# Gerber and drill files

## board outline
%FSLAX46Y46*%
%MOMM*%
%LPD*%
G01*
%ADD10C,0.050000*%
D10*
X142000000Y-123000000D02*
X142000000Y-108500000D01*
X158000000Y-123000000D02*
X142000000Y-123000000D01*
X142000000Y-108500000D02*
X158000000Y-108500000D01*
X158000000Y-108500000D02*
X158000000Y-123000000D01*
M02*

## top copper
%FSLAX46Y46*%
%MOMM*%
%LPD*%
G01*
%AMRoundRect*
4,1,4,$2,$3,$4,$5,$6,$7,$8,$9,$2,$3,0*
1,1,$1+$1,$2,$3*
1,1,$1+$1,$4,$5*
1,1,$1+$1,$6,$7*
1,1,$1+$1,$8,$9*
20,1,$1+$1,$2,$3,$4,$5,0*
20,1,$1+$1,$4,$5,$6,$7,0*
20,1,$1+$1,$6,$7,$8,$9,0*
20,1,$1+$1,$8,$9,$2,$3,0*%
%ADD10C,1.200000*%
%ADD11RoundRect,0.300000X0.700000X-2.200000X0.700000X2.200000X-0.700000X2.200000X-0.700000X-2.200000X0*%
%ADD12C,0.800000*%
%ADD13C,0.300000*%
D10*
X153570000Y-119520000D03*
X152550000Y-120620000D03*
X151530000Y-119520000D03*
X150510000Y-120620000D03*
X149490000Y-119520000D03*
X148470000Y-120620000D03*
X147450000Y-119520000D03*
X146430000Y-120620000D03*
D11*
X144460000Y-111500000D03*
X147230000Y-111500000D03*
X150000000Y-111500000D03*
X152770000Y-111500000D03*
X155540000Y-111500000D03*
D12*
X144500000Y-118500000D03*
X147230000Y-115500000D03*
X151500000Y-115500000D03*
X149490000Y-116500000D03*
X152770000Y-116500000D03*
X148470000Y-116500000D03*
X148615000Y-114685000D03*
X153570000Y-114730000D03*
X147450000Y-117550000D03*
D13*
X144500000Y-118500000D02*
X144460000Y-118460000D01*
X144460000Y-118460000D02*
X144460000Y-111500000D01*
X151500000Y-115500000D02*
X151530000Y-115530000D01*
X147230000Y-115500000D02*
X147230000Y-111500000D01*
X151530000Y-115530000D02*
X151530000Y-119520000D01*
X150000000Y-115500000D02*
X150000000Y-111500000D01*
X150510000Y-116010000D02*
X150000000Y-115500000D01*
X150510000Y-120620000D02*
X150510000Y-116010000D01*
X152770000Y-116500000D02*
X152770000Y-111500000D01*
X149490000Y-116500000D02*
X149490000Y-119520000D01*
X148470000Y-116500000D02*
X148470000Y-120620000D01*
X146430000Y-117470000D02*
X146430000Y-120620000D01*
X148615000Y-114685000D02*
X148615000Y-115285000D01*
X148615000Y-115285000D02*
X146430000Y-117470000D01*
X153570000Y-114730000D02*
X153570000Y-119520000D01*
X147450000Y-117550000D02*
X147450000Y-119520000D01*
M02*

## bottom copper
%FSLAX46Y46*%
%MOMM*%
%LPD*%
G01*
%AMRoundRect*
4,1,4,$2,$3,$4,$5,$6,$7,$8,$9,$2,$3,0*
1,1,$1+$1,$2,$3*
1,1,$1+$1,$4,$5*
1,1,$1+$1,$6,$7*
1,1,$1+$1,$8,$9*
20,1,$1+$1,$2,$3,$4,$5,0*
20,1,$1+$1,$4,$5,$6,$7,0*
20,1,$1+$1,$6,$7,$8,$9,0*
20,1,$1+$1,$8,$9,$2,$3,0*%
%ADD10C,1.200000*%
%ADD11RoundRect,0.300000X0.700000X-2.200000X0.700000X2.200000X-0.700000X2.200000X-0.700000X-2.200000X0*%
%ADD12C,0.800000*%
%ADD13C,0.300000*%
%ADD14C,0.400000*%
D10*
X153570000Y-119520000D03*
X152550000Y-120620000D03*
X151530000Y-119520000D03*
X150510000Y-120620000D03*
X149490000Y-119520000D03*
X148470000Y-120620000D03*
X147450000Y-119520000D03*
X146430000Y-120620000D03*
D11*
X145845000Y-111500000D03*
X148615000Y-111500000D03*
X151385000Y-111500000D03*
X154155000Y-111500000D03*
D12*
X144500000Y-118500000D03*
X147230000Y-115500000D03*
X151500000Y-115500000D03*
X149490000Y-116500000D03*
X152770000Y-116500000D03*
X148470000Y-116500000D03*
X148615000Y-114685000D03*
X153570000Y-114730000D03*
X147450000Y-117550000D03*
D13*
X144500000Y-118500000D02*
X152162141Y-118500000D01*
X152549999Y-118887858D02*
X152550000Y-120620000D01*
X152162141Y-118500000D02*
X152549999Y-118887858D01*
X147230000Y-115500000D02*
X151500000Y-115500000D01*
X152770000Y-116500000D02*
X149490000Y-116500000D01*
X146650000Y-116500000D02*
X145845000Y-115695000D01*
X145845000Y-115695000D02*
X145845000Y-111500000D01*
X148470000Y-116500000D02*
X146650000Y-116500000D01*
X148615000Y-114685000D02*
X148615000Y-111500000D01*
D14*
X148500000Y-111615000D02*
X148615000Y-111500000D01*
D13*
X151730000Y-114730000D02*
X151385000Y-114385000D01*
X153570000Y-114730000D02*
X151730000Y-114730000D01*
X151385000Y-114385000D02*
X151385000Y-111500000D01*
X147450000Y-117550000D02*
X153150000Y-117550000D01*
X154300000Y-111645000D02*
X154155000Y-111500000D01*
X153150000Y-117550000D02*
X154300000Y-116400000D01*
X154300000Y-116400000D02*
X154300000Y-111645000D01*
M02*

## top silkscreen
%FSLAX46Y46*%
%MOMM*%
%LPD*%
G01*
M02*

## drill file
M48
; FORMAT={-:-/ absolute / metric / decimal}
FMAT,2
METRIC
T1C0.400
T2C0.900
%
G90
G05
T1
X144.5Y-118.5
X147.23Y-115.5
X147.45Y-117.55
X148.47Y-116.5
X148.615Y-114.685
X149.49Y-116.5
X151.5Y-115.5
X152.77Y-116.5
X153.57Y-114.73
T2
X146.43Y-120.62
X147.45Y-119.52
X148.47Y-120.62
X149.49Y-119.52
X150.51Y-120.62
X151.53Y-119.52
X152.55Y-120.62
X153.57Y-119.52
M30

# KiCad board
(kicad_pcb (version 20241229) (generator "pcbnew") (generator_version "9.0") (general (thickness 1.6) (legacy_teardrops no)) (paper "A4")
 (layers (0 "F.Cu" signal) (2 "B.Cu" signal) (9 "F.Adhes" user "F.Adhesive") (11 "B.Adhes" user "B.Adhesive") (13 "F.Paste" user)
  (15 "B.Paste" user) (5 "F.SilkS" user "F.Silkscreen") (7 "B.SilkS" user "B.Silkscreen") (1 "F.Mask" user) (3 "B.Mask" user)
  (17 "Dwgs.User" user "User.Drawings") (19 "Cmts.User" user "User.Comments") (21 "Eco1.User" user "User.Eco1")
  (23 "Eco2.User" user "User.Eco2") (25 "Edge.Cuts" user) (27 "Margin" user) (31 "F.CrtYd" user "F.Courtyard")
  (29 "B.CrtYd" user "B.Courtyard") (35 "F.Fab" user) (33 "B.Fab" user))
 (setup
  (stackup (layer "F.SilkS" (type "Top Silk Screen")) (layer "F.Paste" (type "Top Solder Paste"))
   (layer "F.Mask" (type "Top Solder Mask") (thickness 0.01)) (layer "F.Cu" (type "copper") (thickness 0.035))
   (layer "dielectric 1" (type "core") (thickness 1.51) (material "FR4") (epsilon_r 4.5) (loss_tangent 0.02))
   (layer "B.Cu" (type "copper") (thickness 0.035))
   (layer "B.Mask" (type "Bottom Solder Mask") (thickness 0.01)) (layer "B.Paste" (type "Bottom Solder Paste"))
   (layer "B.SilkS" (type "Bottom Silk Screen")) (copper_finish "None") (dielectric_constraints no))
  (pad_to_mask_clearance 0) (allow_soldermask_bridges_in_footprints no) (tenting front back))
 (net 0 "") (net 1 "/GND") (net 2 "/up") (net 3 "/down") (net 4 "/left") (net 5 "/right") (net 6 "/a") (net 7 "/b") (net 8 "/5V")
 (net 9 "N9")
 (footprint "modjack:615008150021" (layer "F.Cu") (at 150 122.5)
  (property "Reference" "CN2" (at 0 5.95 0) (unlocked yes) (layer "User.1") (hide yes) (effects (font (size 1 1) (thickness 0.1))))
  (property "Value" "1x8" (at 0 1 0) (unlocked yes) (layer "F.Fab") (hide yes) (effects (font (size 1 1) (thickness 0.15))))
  (pad "1" thru_hole circle (at 3.57 -2.98) (size 1.2 1.2) (drill 0.9) (layers "*.Cu" "*.Mask") (remove_unused_layers no) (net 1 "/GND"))
  (pad "2" thru_hole circle (at 2.55 -1.88) (size 1.2 1.2) (drill 0.9) (layers "*.Cu" "*.Mask") (remove_unused_layers no) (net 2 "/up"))
  (pad "3" thru_hole circle (at 1.53 -2.98) (size 1.2 1.2) (drill 0.9) (layers "*.Cu" "*.Mask") (remove_unused_layers no) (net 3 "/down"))
  (pad "4" thru_hole circle (at 0.51 -1.88) (size 1.2 1.2) (drill 0.9) (layers "*.Cu" "*.Mask") (remove_unused_layers no) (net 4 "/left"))
  (pad "5" thru_hole circle (at -0.51 -2.98) (size 1.2 1.2) (drill 0.9) (layers "*.Cu" "*.Mask") (remove_unused_layers no) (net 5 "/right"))
  (pad "6" thru_hole circle (at -1.53 -1.88) (size 1.2 1.2) (drill 0.9) (layers "*.Cu" "*.Mask") (remove_unused_layers no) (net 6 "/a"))
  (pad "7" thru_hole circle (at -2.55 -2.98) (size 1.2 1.2) (drill 0.9) (layers "*.Cu" "*.Mask") (remove_unused_layers no) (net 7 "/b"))
  (pad "8" thru_hole circle (at -3.57 -1.88) (size 1.2 1.2) (drill 0.9) (layers "*.Cu" "*.Mask") (remove_unused_layers no) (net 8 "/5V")))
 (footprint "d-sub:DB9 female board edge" (layer "F.Cu") (at 150 111.5 90)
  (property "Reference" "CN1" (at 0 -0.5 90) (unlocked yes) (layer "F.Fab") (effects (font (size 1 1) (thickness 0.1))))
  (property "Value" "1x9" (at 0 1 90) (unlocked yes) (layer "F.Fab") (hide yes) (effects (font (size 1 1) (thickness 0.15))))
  (pad "1" smd roundrect (at 0 -5.54 90) (size 5 2) (layers "F.Cu" "F.Mask" "F.Paste") (roundrect_rratio 0.15) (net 2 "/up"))
  (pad "2" smd roundrect (at 0 -2.77 90) (size 5 2) (layers "F.Cu" "F.Mask" "F.Paste") (roundrect_rratio 0.15) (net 3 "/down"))
  (pad "3" smd roundrect (at 0 0 90) (size 5 2) (layers "F.Cu" "F.Mask" "F.Paste") (roundrect_rratio 0.15) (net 4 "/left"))
  (pad "4" smd roundrect (at 0 2.77 90) (size 5 2) (layers "F.Cu" "F.Mask" "F.Paste") (roundrect_rratio 0.15) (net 5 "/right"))
  (pad "5" smd roundrect (at 0 5.54 90) (size 5 2) (layers "F.Cu" "F.Mask" "F.Paste") (roundrect_rratio 0.15) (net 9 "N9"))
  (pad "6" smd roundrect (at 0 -4.155 90) (size 5 2) (layers "B.Cu" "B.Mask" "B.Paste") (roundrect_rratio 0.15) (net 6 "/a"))
  (pad "7" smd roundrect (at 0 -1.385 90) (size 5 2) (layers "B.Cu" "B.Mask" "B.Paste") (roundrect_rratio 0.15) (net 8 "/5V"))
  (pad "8" smd roundrect (at 0 1.385 90) (size 5 2) (layers "B.Cu" "B.Mask" "B.Paste") (roundrect_rratio 0.15) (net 1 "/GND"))
  (pad "9" smd roundrect (at 0 4.155 90) (size 5 2) (layers "B.Cu" "B.Mask" "B.Paste") (roundrect_rratio 0.15) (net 7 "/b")))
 (gr_line (start 142 123) (end 142 108.5) (stroke (width 0.05) (type solid)) (layer "Edge.Cuts"))
 (gr_line (start 158 123) (end 142 123) (stroke (width 0.05) (type solid)) (layer "Edge.Cuts"))
 (gr_line (start 142 108.5) (end 158 108.5) (stroke (width 0.05) (type solid)) (layer "Edge.Cuts"))
 (gr_line (start 158 108.5) (end 158 123) (stroke (width 0.05) (type solid)) (layer "Edge.Cuts"))
 (segment (start 144.5 118.5) (end 144.46 118.46) (width 0.3) (layer "F.Cu") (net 2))
 (segment (start 144.46 118.46) (end 144.46 111.5) (width 0.3) (layer "F.Cu") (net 2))
 (via (at 144.5 118.5) (size 0.8) (drill 0.4) (layers "F.Cu" "B.Cu") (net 2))
 (segment (start 144.5 118.5) (end 152.162141 118.5) (width 0.3) (layer "B.Cu") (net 2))
 (segment (start 152.549999 118.887858) (end 152.55 120.62) (width 0.3) (layer "B.Cu") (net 2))
 (segment (start 152.162141 118.5) (end 152.549999 118.887858) (width 0.3) (layer "B.Cu") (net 2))
 (segment (start 151.5 115.5) (end 151.53 115.53) (width 0.3) (layer "F.Cu") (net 3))
 (segment (start 147.23 115.5) (end 147.23 111.5) (width 0.3) (layer "F.Cu") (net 3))
 (segment (start 151.53 115.53) (end 151.53 119.52) (width 0.3) (layer "F.Cu") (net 3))
 (via (at 147.23 115.5) (size 0.8) (drill 0.4) (layers "F.Cu" "B.Cu") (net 3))
 (via (at 151.5 115.5) (size 0.8) (drill 0.4) (layers "F.Cu" "B.Cu") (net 3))
 (segment (start 147.23 115.5) (end 151.5 115.5) (width 0.3) (layer "B.Cu") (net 3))
 (segment (start 150 115.5) (end 150 111.5) (width 0.3) (layer "F.Cu") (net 4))
 (segment (start 150.51 116.01) (end 150 115.5) (width 0.3) (layer "F.Cu") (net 4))
 (segment (start 150.51 120.62) (end 150.51 116.01) (width 0.3) (layer "F.Cu") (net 4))
 (segment (start 152.77 116.5) (end 152.77 111.5) (width 0.3) (layer "F.Cu") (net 5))
 (segment (start 149.49 116.5) (end 149.49 119.52) (width 0.3) (layer "F.Cu") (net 5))
 (via (at 149.49 116.5) (size 0.8) (drill 0.4) (layers "F.Cu" "B.Cu") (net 5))
 (via (at 152.77 116.5) (size 0.8) (drill 0.4) (layers "F.Cu" "B.Cu") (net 5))
 (segment (start 152.77 116.5) (end 149.49 116.5) (width 0.3) (layer "B.Cu") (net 5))
 (segment (start 148.47 116.5) (end 148.47 120.62) (width 0.3) (layer "F.Cu") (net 6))
 (via (at 148.47 116.5) (size 0.8) (drill 0.4) (layers "F.Cu" "B.Cu") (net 6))
 (segment (start 146.65 116.5) (end 145.845 115.695) (width 0.3) (layer "B.Cu") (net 6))
 (segment (start 145.845 115.695) (end 145.845 111.5) (width 0.3) (layer "B.Cu") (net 6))
 (segment (start 148.47 116.5) (end 146.65 116.5) (width 0.3) (layer "B.Cu") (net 6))
 (segment (start 146.43 117.47) (end 146.43 120.62) (width 0.3) (layer "F.Cu") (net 8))
 (segment (start 148.615 114.685) (end 148.615 115.285) (width 0.3) (layer "F.Cu") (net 8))
 (segment (start 148.615 115.285) (end 146.43 117.47) (width 0.3) (layer "F.Cu") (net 8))
 (via (at 148.615 114.685) (size 0.8) (drill 0.4) (layers "F.Cu" "B.Cu") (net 8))
 (segment (start 148.615 114.685) (end 148.615 111.5) (width 0.3) (layer "B.Cu") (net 8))
 (segment (start 148.5 111.615) (end 148.615 111.5) (width 0.4) (layer "B.Cu") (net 8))
 (segment (start 153.57 114.73) (end 153.57 119.52) (width 0.3) (layer "F.Cu") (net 1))
 (via (at 153.57 114.73) (size 0.8) (drill 0.4) (layers "F.Cu" "B.Cu") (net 1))
 (segment (start 151.73 114.73) (end 151.385 114.385) (width 0.3) (layer "B.Cu") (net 1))
 (segment (start 153.57 114.73) (end 151.73 114.73) (width 0.3) (layer "B.Cu") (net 1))
 (segment (start 151.385 114.385) (end 151.385 111.5) (width 0.3) (layer "B.Cu") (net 1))
 (segment (start 147.45 117.55) (end 147.45 119.52) (width 0.3) (layer "F.Cu") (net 7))
 (via (at 147.45 117.55) (size 0.8) (drill 0.4) (layers "F.Cu" "B.Cu") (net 7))
 (segment (start 147.45 117.55) (end 153.15 117.55) (width 0.3) (layer "B.Cu") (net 7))
 (segment (start 154.3 111.645) (end 154.155 111.5) (width 0.3) (layer "B.Cu") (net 7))
 (segment (start 153.15 117.55) (end 154.3 116.4) (width 0.3) (layer "B.Cu") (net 7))
 (segment (start 154.3 116.4) (end 154.3 111.645) (width 0.3) (layer "B.Cu") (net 7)))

